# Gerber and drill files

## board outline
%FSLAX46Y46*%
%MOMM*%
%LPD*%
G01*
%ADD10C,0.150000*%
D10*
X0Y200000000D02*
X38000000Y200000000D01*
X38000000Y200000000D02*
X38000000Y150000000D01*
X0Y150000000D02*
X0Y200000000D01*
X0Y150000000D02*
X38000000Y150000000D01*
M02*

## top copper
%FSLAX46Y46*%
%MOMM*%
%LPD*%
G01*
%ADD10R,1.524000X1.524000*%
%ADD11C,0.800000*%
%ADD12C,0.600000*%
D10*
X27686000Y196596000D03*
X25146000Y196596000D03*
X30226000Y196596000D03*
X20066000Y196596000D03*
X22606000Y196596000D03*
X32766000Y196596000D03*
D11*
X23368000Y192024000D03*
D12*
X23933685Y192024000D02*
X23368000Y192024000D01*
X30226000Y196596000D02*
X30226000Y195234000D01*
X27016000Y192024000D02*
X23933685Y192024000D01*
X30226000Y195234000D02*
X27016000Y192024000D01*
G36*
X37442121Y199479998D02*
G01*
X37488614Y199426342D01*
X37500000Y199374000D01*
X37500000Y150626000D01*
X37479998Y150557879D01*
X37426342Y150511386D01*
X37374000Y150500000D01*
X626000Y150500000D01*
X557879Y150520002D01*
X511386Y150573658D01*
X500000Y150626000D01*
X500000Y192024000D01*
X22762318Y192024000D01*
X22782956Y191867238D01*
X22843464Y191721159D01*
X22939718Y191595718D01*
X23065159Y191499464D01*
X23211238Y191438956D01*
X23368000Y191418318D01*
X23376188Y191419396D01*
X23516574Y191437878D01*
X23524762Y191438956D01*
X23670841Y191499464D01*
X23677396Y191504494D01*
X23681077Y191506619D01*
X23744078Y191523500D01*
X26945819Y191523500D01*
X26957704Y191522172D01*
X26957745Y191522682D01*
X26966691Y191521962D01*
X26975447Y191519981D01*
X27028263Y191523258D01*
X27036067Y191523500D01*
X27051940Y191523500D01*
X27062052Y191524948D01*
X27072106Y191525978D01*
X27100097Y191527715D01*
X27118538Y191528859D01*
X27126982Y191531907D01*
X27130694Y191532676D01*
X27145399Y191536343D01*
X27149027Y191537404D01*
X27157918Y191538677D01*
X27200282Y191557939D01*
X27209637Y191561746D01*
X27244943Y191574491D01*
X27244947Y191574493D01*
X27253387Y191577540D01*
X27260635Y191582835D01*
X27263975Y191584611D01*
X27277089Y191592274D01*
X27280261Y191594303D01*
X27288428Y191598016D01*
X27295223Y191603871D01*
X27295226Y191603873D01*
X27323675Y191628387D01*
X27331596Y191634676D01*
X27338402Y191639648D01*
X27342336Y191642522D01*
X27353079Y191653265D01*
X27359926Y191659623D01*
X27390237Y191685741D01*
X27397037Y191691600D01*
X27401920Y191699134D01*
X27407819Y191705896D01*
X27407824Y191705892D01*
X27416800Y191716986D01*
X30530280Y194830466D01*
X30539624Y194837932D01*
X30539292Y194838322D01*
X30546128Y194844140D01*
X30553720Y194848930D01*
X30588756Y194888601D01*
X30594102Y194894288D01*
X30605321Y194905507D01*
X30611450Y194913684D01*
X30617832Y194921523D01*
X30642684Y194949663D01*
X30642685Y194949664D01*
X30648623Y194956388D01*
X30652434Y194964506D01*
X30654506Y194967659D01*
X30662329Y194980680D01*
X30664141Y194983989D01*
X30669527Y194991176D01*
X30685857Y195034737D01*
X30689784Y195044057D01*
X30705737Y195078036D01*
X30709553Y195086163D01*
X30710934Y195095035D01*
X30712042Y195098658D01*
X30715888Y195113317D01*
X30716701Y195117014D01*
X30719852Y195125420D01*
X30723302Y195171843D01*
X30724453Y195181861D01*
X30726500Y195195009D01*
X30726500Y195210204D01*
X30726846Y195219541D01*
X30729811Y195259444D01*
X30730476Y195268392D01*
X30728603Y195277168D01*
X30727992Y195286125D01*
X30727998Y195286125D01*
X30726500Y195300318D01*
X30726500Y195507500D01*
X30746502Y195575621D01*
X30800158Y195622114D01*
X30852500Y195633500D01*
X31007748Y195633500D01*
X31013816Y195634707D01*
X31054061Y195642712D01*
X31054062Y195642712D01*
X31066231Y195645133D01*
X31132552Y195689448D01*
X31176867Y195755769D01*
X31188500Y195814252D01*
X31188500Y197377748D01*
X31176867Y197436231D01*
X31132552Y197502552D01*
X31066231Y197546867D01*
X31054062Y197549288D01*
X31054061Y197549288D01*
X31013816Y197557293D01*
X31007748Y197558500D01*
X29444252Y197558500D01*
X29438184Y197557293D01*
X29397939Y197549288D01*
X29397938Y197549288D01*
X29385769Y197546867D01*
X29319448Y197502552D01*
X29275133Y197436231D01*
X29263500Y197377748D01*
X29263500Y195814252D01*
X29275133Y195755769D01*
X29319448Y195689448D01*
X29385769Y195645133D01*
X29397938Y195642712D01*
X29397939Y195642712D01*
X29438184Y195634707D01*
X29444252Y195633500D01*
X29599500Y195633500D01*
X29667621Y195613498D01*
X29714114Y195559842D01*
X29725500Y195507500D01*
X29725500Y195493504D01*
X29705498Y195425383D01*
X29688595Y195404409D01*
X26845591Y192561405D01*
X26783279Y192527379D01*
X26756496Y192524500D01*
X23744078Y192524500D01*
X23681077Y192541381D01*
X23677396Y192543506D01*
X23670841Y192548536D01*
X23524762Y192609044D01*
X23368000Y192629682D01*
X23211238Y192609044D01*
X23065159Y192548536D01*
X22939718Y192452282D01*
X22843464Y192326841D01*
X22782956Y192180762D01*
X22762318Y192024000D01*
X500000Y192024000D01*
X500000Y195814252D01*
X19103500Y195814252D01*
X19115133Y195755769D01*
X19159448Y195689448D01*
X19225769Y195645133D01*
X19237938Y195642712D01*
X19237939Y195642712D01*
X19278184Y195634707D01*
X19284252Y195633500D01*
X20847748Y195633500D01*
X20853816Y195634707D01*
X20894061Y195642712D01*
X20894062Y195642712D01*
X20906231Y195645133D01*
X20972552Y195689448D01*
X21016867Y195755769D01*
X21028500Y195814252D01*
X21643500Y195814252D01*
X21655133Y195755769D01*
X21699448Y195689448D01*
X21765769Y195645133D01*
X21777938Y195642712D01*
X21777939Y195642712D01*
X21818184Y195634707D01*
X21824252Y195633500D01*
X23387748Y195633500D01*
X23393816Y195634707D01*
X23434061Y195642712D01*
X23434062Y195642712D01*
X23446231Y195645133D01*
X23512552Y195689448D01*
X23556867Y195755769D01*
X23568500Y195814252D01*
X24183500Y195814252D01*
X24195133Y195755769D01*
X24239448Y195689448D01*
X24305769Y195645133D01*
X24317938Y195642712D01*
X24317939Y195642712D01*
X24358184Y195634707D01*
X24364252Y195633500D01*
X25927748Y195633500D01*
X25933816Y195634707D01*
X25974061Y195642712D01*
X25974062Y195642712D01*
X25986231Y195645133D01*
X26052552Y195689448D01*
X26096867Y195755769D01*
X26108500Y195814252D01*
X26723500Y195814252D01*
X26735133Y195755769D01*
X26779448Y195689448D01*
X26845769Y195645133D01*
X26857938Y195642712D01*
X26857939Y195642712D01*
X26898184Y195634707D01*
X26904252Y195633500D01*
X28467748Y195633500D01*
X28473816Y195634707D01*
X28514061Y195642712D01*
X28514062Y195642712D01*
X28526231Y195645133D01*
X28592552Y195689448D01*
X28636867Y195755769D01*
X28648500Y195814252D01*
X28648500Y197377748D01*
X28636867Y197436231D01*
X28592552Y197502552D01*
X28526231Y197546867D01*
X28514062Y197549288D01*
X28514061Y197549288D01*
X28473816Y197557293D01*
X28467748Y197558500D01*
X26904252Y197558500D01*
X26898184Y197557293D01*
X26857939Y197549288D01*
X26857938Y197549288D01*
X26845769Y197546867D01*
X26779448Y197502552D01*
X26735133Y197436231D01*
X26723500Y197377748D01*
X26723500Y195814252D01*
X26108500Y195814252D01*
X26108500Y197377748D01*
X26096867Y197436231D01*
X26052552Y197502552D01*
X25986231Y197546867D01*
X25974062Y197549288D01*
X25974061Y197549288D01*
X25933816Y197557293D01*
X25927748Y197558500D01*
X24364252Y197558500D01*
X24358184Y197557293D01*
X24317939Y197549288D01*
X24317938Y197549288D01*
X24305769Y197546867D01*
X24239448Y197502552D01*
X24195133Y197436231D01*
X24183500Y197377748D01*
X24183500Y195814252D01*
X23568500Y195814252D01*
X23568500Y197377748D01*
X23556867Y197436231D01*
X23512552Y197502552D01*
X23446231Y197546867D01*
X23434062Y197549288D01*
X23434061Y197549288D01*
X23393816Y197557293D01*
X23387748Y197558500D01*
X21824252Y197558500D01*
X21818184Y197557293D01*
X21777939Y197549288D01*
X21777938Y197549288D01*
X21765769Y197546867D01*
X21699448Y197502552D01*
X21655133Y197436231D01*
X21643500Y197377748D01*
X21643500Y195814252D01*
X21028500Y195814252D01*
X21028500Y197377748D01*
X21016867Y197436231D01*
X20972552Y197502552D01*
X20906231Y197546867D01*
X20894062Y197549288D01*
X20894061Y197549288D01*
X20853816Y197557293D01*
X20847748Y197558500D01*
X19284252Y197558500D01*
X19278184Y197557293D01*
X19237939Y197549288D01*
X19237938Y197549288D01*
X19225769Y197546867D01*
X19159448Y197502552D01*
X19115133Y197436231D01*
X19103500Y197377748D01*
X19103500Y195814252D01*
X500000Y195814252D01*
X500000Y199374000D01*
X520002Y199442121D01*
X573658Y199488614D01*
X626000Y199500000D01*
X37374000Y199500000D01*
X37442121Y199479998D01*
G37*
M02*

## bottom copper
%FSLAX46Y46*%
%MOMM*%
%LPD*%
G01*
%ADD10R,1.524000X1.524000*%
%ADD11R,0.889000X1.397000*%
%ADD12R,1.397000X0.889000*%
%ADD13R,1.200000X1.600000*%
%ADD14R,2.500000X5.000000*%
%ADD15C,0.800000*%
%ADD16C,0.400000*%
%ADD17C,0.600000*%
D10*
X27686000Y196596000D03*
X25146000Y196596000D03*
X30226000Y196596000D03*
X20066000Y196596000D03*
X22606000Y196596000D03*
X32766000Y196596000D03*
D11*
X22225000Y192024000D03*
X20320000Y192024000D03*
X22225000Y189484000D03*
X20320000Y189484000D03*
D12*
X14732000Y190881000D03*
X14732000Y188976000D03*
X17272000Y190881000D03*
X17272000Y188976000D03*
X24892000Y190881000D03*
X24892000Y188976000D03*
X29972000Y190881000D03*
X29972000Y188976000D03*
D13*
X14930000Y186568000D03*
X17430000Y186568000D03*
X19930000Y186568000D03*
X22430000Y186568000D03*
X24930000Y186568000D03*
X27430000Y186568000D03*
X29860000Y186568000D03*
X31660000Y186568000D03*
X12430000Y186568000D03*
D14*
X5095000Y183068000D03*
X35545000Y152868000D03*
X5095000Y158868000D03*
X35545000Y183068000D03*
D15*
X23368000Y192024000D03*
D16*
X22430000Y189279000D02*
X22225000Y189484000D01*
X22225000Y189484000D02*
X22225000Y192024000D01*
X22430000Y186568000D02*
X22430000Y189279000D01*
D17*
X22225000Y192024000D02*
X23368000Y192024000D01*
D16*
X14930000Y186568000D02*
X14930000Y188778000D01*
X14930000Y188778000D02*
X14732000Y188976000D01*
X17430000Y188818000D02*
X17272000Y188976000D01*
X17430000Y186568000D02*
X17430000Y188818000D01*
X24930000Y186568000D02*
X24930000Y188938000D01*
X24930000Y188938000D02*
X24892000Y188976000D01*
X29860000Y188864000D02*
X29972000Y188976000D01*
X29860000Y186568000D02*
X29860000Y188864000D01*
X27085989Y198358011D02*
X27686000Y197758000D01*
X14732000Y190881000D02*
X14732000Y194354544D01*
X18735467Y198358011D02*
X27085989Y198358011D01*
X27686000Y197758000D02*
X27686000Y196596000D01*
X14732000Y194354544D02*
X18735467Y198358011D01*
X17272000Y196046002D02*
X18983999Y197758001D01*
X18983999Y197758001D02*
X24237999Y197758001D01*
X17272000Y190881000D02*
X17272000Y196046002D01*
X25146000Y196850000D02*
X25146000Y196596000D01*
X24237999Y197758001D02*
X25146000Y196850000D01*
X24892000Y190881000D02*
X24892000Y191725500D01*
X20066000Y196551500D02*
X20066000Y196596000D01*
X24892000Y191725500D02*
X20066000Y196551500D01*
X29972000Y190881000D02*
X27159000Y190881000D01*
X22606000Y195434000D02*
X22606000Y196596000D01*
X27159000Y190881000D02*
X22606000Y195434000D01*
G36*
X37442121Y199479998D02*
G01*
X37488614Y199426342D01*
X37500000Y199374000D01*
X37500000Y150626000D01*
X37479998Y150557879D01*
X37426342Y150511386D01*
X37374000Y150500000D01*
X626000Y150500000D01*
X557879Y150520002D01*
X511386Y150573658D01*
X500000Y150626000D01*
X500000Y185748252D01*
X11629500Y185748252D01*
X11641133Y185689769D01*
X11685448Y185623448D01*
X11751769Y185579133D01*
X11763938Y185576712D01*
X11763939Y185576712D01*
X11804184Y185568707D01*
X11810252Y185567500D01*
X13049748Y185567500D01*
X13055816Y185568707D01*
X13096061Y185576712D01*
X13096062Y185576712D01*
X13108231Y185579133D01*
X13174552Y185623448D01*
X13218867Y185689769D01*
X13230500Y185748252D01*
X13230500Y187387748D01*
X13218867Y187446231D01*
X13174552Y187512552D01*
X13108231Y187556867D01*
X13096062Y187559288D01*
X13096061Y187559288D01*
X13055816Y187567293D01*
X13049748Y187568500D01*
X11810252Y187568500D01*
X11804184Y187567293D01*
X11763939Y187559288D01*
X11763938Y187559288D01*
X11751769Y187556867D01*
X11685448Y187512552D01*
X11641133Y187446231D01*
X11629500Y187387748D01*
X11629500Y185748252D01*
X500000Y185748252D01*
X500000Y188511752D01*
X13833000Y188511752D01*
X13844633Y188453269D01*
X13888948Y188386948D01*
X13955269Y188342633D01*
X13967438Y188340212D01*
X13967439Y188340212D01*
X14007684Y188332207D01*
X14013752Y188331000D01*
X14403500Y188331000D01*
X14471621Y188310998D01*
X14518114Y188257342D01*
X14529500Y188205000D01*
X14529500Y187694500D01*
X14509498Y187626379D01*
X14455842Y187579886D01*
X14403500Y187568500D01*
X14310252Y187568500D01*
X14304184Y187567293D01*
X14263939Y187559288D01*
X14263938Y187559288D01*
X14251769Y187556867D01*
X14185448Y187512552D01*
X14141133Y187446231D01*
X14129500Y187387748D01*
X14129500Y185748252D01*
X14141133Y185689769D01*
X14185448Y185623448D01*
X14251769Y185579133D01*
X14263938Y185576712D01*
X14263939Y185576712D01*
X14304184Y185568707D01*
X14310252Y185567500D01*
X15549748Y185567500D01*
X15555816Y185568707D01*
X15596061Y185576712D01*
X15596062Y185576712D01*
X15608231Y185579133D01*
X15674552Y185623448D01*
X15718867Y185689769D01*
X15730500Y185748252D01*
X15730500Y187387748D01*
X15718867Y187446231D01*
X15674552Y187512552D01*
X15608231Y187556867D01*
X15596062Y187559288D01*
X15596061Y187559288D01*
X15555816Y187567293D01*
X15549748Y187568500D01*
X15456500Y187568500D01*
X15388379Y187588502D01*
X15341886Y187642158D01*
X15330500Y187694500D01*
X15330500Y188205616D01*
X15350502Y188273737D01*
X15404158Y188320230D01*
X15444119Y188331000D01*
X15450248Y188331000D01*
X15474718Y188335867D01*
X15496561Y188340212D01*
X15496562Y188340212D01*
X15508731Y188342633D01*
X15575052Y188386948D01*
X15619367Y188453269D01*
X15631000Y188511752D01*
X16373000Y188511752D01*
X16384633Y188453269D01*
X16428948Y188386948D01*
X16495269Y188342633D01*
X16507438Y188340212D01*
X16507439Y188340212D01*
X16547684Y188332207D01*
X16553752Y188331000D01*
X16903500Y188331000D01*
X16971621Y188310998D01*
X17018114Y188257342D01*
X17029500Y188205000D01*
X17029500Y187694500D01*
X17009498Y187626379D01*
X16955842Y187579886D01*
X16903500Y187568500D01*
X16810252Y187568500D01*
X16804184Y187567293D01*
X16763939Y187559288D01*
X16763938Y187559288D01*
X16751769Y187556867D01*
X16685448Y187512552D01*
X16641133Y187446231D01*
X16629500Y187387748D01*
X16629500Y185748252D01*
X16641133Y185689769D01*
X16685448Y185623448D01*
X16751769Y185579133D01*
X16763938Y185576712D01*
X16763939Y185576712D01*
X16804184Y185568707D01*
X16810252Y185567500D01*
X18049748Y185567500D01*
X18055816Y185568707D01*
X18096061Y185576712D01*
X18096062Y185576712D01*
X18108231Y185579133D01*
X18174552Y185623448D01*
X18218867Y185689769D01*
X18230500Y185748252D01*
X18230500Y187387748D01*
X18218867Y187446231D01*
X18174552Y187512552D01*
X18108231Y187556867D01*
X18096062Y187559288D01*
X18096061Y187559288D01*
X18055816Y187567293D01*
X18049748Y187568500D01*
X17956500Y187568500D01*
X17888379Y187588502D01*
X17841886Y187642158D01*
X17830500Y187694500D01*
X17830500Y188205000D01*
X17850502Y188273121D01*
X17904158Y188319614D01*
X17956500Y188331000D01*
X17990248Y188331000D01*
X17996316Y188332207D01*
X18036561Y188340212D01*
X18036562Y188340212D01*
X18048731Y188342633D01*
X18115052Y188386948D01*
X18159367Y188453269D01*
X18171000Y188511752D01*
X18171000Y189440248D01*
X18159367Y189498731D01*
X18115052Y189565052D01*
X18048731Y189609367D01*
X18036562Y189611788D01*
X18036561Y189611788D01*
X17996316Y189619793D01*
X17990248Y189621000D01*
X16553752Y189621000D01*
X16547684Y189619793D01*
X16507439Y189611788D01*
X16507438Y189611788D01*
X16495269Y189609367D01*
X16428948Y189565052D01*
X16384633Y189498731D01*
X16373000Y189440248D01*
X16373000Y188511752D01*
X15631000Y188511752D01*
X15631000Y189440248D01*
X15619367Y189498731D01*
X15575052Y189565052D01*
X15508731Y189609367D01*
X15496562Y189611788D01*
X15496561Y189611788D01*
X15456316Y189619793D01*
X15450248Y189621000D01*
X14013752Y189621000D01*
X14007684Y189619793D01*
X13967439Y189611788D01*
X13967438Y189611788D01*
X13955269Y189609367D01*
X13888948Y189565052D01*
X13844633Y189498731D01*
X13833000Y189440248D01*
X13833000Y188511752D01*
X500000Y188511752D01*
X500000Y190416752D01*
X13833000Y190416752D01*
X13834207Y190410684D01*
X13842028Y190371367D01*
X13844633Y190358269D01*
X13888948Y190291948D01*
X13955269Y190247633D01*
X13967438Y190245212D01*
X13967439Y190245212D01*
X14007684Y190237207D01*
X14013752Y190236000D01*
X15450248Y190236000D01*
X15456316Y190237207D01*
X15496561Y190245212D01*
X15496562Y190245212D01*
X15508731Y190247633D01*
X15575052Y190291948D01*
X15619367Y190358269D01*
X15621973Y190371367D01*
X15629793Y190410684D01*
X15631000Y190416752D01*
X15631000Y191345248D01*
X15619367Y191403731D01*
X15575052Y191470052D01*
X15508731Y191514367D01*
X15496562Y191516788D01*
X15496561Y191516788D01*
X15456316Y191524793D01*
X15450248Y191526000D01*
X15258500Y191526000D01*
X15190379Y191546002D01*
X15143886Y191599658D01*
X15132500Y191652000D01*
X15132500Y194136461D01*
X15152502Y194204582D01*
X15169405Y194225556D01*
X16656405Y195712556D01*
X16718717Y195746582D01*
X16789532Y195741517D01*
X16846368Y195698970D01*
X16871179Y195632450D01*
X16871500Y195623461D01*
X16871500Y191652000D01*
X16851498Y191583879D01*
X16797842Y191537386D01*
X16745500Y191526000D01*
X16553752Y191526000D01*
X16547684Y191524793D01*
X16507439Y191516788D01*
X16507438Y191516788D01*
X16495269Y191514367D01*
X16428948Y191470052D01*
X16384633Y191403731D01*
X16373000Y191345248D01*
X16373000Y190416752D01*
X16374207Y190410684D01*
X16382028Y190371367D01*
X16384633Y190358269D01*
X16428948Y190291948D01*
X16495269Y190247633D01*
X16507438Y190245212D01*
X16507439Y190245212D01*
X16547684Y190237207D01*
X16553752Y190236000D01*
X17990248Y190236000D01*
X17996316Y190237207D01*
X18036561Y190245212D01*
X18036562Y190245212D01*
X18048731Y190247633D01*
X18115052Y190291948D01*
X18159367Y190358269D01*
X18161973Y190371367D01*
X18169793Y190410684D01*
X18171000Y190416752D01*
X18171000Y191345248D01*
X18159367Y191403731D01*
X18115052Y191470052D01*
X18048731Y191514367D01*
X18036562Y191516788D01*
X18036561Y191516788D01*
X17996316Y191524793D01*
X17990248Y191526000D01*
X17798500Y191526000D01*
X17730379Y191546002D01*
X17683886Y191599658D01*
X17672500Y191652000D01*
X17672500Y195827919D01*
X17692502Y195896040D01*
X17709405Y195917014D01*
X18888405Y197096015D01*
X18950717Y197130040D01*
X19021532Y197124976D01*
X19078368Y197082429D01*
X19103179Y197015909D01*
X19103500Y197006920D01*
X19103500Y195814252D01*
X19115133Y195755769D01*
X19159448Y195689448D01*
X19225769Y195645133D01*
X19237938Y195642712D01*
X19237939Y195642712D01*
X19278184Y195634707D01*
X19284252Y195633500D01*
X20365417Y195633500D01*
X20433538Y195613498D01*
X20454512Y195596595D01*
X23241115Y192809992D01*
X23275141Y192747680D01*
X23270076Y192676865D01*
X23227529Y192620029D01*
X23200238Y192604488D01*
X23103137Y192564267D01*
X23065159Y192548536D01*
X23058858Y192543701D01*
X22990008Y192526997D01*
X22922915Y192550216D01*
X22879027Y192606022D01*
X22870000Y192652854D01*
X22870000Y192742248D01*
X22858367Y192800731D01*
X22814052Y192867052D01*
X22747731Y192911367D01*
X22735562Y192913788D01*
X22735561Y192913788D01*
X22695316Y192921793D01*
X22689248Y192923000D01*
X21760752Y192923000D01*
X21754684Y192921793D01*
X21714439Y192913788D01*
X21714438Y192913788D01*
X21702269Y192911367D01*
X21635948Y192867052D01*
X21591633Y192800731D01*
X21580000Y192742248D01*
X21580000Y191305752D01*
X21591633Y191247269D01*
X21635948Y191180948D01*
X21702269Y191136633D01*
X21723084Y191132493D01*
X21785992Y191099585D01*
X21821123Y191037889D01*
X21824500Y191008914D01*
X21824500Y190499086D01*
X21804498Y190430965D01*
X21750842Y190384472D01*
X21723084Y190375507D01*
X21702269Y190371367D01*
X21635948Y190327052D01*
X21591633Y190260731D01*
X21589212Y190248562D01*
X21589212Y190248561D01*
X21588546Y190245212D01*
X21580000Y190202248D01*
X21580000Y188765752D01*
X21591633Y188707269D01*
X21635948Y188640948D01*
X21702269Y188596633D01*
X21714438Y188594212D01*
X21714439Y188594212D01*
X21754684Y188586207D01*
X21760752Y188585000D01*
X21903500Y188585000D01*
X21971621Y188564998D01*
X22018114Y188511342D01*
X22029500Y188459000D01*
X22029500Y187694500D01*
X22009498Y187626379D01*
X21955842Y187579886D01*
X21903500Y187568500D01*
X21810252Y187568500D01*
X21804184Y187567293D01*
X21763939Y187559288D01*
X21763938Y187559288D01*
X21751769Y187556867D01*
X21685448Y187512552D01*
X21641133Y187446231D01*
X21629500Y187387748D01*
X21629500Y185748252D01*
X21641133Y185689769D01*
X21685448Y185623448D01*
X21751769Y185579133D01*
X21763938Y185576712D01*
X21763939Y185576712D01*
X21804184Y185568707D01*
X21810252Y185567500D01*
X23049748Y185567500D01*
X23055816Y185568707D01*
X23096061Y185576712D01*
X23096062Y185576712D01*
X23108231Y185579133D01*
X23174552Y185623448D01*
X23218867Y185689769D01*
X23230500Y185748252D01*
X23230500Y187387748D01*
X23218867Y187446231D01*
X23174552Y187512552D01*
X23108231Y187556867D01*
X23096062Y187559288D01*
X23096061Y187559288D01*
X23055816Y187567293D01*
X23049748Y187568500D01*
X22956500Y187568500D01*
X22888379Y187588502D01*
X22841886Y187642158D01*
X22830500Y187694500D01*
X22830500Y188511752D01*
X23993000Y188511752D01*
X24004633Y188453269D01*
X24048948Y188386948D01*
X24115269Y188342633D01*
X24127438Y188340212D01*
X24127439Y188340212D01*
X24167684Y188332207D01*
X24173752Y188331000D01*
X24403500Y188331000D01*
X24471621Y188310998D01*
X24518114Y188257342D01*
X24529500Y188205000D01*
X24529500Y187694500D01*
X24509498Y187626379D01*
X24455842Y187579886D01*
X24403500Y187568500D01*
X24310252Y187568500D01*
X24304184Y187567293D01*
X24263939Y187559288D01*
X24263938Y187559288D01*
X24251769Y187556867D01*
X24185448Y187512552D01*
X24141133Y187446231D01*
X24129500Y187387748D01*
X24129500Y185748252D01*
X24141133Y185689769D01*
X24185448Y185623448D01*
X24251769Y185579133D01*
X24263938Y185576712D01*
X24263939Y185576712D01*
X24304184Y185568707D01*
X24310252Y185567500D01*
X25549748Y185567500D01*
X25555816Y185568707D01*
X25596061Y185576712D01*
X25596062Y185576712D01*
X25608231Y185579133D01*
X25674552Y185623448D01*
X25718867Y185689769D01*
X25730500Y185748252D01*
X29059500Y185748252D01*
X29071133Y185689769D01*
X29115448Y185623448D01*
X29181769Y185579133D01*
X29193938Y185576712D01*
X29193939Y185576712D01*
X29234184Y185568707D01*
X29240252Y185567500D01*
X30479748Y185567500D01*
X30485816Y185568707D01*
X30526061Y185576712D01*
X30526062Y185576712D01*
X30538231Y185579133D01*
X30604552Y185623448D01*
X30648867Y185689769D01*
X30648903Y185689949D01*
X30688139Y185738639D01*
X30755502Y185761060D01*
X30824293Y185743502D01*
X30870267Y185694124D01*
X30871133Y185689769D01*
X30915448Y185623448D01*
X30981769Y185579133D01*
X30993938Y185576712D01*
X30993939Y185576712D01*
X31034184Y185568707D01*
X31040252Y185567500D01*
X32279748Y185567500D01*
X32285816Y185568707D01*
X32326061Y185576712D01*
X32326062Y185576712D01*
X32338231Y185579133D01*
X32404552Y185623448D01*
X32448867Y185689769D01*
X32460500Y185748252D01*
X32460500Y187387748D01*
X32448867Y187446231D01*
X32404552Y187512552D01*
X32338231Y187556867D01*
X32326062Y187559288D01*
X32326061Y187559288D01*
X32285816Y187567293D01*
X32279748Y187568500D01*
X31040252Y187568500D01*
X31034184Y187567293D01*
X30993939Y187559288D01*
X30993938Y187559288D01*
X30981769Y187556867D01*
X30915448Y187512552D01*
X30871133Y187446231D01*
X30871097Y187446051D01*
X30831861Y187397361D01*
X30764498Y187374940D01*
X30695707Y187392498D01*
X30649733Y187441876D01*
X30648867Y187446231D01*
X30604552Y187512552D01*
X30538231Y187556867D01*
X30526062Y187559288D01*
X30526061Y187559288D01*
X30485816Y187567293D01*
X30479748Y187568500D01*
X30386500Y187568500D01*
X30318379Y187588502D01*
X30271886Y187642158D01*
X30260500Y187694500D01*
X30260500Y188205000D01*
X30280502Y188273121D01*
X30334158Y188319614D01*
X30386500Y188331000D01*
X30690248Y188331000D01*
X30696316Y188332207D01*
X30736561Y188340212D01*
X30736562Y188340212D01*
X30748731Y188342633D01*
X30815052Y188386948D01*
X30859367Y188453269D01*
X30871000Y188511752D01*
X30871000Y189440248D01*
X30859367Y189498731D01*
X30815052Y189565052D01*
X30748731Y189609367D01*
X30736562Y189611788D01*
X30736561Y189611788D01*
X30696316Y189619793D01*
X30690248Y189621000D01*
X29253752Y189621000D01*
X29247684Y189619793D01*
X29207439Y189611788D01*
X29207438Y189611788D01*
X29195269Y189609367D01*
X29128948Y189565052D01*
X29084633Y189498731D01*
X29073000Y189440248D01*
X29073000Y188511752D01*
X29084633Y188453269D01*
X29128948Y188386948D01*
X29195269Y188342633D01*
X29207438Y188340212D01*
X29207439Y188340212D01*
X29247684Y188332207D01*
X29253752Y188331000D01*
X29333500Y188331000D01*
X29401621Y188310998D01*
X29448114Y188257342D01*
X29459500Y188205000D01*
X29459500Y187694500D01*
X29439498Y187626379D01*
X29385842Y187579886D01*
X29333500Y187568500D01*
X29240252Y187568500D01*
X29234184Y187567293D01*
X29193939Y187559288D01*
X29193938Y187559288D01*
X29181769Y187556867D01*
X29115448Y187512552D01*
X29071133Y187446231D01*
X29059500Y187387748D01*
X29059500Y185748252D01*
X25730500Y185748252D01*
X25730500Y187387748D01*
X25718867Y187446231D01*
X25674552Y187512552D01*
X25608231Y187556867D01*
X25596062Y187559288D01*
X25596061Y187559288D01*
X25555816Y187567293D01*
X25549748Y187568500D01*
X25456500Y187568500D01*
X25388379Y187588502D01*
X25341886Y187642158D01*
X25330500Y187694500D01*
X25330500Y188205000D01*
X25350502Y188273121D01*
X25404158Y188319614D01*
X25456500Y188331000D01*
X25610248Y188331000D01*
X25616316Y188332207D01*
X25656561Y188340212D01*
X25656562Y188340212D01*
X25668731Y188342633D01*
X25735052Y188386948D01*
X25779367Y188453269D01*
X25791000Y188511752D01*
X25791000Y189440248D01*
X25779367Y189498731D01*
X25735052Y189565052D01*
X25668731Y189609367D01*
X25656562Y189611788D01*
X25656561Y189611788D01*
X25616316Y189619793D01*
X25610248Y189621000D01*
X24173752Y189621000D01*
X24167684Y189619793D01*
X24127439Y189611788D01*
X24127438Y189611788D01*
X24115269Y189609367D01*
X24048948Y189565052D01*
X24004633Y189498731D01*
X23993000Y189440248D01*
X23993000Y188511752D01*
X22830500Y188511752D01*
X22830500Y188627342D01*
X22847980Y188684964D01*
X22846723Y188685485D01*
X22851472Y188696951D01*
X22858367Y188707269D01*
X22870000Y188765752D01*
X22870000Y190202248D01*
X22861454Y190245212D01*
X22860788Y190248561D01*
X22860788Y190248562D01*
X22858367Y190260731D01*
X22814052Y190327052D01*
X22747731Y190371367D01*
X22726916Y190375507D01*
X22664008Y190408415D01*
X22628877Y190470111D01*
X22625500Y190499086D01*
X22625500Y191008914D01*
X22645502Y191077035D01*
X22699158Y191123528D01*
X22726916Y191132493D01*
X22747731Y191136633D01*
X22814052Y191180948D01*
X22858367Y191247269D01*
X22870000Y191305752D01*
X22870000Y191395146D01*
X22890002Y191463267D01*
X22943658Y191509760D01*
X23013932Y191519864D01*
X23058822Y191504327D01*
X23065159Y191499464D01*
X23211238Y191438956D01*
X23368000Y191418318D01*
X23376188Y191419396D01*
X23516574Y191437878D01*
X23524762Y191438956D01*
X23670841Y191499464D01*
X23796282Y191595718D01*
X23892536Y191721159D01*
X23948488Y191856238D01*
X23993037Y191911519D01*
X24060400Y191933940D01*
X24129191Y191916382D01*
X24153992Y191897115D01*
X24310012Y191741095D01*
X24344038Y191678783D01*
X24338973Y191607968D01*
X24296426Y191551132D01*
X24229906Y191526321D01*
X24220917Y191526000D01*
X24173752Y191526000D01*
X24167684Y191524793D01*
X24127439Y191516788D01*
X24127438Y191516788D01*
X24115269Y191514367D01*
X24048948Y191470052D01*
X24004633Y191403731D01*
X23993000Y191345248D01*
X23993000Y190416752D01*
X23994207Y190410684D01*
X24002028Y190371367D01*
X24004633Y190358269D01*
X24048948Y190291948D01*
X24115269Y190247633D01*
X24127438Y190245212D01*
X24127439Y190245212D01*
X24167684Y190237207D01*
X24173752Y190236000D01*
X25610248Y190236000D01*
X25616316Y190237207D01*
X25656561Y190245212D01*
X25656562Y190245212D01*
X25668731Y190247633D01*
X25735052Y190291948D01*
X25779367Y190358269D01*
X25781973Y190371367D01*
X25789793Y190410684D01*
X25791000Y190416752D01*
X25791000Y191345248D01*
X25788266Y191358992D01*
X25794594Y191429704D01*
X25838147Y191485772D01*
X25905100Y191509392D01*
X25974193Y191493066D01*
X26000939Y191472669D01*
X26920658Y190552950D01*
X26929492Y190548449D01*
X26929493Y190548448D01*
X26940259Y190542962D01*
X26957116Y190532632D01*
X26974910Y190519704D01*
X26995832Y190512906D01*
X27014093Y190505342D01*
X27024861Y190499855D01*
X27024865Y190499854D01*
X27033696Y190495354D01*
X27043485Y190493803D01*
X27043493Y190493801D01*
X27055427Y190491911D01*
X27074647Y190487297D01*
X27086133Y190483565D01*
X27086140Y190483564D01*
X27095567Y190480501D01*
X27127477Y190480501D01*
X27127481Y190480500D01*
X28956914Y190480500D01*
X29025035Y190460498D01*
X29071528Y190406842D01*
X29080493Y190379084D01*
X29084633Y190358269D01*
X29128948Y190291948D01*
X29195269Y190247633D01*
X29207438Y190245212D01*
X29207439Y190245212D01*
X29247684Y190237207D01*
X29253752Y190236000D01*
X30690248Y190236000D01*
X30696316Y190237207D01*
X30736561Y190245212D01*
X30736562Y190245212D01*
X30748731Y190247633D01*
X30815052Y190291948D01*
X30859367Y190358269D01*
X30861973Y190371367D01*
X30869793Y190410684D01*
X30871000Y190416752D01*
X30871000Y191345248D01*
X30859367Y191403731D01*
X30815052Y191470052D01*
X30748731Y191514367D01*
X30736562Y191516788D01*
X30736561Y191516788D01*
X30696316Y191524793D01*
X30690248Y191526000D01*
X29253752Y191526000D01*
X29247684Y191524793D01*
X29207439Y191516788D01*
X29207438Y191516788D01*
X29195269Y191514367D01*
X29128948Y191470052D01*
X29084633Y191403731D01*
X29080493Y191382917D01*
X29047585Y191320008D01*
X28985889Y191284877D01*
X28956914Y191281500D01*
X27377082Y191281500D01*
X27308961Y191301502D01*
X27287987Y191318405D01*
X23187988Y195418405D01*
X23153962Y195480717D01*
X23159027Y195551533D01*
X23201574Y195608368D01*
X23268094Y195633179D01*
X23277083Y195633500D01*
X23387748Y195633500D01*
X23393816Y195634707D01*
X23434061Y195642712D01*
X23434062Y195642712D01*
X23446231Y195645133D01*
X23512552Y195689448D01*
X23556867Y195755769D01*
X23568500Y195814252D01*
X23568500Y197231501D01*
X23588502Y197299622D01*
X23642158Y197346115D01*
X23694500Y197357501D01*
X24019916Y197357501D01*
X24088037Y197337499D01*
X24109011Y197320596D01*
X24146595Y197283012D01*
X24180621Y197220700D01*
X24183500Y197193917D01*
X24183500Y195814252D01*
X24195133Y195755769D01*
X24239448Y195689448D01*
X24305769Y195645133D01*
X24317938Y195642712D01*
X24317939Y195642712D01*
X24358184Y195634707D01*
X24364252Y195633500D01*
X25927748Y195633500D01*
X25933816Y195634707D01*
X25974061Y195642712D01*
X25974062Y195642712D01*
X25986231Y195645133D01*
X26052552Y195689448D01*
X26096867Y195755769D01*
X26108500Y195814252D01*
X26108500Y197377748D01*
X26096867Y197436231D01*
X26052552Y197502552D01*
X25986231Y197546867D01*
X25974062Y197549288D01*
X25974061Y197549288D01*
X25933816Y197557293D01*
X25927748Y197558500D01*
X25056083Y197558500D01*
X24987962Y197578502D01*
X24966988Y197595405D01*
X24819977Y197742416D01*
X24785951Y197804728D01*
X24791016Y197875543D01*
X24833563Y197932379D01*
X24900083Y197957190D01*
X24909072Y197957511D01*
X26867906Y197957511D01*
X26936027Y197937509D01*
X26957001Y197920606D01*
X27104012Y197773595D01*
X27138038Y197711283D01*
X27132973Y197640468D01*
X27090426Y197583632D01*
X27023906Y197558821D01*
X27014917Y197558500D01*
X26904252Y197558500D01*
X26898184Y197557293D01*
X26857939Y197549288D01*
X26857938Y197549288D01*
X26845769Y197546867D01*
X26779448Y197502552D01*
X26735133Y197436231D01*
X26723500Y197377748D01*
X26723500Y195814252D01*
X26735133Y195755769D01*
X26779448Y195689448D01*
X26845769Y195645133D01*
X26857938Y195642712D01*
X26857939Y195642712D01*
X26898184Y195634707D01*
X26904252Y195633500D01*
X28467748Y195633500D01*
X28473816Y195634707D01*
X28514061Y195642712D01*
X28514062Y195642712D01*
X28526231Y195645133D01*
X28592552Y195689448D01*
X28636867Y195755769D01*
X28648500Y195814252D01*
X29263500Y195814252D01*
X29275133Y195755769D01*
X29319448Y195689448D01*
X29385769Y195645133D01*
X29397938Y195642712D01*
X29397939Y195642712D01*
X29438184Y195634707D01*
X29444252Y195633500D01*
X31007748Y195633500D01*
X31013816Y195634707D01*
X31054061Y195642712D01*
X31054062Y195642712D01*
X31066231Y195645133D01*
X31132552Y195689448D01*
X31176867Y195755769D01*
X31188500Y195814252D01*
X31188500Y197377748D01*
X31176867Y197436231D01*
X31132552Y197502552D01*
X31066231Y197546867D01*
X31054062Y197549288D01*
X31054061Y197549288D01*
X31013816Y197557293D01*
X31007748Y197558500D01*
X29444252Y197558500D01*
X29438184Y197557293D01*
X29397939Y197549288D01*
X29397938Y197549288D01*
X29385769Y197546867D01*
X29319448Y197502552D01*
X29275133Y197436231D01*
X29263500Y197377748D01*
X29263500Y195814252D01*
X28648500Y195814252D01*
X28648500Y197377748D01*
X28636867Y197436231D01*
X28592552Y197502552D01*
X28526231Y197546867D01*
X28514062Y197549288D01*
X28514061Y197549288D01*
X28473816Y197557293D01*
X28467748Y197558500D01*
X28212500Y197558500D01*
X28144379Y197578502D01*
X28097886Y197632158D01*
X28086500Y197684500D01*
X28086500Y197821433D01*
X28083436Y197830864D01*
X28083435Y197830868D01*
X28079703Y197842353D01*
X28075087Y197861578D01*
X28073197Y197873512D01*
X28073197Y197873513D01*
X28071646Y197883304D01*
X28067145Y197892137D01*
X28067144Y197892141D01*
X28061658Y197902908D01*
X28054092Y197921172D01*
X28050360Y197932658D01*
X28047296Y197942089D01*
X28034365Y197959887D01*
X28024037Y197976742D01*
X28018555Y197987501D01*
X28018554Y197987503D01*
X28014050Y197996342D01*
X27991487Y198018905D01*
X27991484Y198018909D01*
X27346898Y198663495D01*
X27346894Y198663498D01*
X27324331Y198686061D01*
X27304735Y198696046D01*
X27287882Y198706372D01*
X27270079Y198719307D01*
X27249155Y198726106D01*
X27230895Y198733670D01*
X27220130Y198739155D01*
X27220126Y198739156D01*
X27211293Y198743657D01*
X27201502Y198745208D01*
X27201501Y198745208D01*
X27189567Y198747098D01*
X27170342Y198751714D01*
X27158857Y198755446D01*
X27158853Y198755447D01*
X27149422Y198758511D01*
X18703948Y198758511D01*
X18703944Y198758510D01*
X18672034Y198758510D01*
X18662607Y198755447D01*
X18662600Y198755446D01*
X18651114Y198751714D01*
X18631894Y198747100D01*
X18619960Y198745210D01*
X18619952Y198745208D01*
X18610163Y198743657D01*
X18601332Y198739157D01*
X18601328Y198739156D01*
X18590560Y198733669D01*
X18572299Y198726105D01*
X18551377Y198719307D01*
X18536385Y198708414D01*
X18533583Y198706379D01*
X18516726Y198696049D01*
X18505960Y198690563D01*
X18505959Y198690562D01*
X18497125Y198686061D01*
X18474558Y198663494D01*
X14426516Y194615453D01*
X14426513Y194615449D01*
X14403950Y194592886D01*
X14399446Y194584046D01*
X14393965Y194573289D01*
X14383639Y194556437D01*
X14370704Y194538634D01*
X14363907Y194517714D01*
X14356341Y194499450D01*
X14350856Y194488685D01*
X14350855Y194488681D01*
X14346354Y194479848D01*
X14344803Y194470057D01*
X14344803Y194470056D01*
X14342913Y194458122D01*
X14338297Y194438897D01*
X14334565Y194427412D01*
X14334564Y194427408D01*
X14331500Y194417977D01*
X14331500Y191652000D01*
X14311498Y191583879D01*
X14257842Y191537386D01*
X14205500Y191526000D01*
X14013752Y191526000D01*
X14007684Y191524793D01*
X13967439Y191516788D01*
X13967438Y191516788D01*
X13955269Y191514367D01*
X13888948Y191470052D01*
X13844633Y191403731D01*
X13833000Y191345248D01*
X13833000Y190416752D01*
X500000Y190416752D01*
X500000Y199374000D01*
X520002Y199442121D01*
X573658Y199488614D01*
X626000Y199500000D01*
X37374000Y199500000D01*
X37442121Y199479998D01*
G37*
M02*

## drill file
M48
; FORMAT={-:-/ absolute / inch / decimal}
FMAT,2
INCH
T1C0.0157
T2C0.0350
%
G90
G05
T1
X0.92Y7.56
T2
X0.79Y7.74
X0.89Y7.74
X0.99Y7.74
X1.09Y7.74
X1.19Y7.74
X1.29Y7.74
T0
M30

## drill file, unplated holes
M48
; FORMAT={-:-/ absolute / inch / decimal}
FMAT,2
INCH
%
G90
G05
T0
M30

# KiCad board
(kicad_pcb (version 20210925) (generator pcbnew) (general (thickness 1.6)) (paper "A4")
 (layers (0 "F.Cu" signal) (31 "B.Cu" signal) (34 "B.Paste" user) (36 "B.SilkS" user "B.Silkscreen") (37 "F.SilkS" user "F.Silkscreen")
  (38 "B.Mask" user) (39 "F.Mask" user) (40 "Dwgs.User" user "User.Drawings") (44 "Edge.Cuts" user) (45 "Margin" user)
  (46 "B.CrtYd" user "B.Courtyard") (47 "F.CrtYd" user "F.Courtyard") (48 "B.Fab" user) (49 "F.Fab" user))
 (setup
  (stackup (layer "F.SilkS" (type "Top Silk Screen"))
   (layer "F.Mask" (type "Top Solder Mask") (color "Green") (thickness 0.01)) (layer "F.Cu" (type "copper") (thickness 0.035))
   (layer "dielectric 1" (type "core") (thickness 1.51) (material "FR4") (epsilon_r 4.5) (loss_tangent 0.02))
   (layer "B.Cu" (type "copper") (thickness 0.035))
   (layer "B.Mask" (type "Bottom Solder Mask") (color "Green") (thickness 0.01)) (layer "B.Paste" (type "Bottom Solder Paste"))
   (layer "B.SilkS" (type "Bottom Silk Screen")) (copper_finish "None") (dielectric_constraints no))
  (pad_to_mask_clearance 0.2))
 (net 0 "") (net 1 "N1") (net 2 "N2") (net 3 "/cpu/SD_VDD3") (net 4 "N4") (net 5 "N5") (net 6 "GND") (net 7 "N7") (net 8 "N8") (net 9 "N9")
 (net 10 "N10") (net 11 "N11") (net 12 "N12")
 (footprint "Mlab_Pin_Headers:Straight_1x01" (layer "F.Cu") (at 27.686 -196.596)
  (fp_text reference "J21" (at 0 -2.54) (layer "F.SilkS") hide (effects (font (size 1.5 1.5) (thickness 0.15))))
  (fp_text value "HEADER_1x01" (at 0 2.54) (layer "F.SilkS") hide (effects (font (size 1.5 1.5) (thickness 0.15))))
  (pad "1" thru_hole rect locked (at 0 0) (size 1.524 1.524) (drill 0.889) (layers *.Cu *.Mask "F.SilkS") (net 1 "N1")))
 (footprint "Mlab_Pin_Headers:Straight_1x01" (layer "F.Cu") (at 25.146 -196.596)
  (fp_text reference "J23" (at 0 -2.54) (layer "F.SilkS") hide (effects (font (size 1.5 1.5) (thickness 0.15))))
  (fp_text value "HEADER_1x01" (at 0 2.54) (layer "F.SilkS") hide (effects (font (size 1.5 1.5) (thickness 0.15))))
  (pad "1" thru_hole rect locked (at 0 0) (size 1.524 1.524) (drill 0.889) (layers *.Cu *.Mask "F.SilkS") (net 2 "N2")))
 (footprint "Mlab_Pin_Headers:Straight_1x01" (layer "F.Cu") (at 30.226 -196.596)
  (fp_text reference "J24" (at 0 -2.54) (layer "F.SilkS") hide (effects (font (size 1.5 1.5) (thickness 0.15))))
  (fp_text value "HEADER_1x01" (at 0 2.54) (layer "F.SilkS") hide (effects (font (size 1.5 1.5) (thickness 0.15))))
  (pad "1" thru_hole rect locked (at 0 0) (size 1.524 1.524) (drill 0.889) (layers *.Cu *.Mask "F.SilkS") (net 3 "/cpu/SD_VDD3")))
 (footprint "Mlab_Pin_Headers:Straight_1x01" (layer "F.Cu") (at 20.066 -196.596)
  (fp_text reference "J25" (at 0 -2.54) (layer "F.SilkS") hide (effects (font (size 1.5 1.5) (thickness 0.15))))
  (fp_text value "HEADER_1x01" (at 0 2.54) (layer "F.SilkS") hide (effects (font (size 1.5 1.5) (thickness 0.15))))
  (pad "1" thru_hole rect locked (at 0 0) (size 1.524 1.524) (drill 0.889) (layers *.Cu *.Mask "F.SilkS") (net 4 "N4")))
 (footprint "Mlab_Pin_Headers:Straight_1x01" (layer "F.Cu") (at 22.606 -196.596)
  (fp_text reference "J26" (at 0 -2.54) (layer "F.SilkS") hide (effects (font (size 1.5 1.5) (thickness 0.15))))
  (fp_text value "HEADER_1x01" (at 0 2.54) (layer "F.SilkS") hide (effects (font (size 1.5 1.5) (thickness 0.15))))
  (pad "1" thru_hole rect locked (at 0 0) (size 1.524 1.524) (drill 0.889) (layers *.Cu *.Mask "F.SilkS") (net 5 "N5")))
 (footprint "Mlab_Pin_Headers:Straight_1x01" (layer "F.Cu") (at 32.766 -196.596 90)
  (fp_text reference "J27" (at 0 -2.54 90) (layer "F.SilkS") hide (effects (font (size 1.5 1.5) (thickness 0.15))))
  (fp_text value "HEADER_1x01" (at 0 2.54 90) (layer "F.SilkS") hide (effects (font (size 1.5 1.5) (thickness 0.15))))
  (pad "1" thru_hole rect locked (at 0 0 90) (size 1.524 1.524) (drill 0.889) (layers *.Cu *.Mask "F.SilkS") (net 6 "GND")))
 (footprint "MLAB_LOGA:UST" (layer "F.Cu") (at 18.415 -175.133)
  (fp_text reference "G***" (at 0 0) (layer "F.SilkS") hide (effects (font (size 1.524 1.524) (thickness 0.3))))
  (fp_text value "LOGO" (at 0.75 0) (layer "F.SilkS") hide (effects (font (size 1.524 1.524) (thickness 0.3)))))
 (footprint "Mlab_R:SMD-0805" (layer "B.Cu") (at 21.2725 -192.024 180)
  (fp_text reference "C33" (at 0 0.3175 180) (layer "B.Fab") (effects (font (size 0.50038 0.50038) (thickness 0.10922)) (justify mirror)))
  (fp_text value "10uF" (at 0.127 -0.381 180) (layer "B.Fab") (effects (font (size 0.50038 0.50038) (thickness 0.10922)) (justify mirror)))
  (pad "1" smd rect locked (at -0.9525 0 180) (size 0.889 1.397) (layers "B.Cu" "B.Paste" "B.Mask") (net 3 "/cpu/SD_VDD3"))
  (pad "2" smd rect locked (at 0.9525 0 180) (size 0.889 1.397) (layers "B.Cu" "B.Paste" "B.Mask") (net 6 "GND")))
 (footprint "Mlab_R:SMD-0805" (layer "B.Cu") (at 21.2725 -189.484 180)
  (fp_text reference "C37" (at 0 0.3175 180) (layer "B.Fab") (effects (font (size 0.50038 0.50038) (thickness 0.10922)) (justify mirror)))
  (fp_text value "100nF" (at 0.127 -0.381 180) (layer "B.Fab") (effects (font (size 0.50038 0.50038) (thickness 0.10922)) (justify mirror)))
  (pad "1" smd rect locked (at -0.9525 0 180) (size 0.889 1.397) (layers "B.Cu" "B.Paste" "B.Mask") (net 3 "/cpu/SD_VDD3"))
  (pad "2" smd rect locked (at 0.9525 0 180) (size 0.889 1.397) (layers "B.Cu" "B.Paste" "B.Mask") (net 6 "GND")))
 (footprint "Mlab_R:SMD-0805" (layer "B.Cu") (at 14.732 -189.9285 -90)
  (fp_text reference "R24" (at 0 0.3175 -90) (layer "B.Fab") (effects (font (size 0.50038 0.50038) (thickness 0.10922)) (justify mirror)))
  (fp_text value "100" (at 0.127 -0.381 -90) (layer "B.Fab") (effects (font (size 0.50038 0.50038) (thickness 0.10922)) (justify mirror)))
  (pad "1" smd rect locked (at -0.9525 0 270) (size 0.889 1.397) (layers "B.Cu" "B.Paste" "B.Mask") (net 1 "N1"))
  (pad "2" smd rect locked (at 0.9525 0 270) (size 0.889 1.397) (layers "B.Cu" "B.Paste" "B.Mask") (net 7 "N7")))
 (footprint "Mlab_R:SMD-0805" (layer "B.Cu") (at 17.272 -189.9285 -90)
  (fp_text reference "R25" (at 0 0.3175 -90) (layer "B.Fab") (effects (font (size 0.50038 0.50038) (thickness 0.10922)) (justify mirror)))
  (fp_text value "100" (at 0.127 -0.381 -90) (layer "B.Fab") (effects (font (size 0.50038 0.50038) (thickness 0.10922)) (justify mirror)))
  (pad "1" smd rect locked (at -0.9525 0 270) (size 0.889 1.397) (layers "B.Cu" "B.Paste" "B.Mask") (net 2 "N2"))
  (pad "2" smd rect locked (at 0.9525 0 270) (size 0.889 1.397) (layers "B.Cu" "B.Paste" "B.Mask") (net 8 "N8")))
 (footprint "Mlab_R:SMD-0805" (layer "B.Cu") (at 24.892 -189.9285 -90)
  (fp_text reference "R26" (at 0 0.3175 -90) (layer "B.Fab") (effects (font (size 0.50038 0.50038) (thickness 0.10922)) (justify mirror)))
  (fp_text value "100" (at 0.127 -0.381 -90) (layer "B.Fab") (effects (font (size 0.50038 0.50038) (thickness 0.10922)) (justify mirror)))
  (pad "1" smd rect locked (at -0.9525 0 270) (size 0.889 1.397) (layers "B.Cu" "B.Paste" "B.Mask") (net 4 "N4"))
  (pad "2" smd rect locked (at 0.9525 0 270) (size 0.889 1.397) (layers "B.Cu" "B.Paste" "B.Mask") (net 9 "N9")))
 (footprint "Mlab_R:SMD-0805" (layer "B.Cu") (at 29.972 -189.9285 -90)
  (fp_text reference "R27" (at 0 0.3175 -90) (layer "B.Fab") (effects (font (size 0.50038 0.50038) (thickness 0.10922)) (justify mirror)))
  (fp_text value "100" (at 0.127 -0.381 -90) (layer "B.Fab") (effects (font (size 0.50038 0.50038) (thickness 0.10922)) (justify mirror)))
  (pad "1" smd rect locked (at -0.9525 0 270) (size 0.889 1.397) (layers "B.Cu" "B.Paste" "B.Mask") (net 5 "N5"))
  (pad "2" smd rect locked (at 0.9525 0 270) (size 0.889 1.397) (layers "B.Cu" "B.Paste" "B.Mask") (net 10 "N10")))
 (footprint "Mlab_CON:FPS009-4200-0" (layer "B.Cu") (at 20.32 -150.368 -90)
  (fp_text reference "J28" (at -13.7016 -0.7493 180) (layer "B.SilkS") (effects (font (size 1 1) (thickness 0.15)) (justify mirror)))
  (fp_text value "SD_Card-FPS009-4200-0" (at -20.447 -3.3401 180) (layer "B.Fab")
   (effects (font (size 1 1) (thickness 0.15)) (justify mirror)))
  (pad "1" smd rect locked (at -36.2 5.39 90) (size 1.6 1.2) (layers "B.Cu" "B.Paste" "B.Mask") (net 7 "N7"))
  (pad "2" smd rect locked (at -36.2 2.89 90) (size 1.6 1.2) (layers "B.Cu" "B.Paste" "B.Mask") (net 8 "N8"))
  (pad "3" smd rect locked (at -36.2 0.39 90) (size 1.6 1.2) (layers "B.Cu" "B.Paste" "B.Mask") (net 6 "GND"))
  (pad "4" smd rect locked (at -36.2 -2.11 90) (size 1.6 1.2) (layers "B.Cu" "B.Paste" "B.Mask") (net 3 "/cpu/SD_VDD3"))
  (pad "5" smd rect locked (at -36.2 -4.61 90) (size 1.6 1.2) (layers "B.Cu" "B.Paste" "B.Mask") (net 9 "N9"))
  (pad "6" smd rect locked (at -36.2 -7.11 90) (size 1.6 1.2) (layers "B.Cu" "B.Paste" "B.Mask") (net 6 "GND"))
  (pad "7" smd rect locked (at -36.2 -9.54 90) (size 1.6 1.2) (layers "B.Cu" "B.Paste" "B.Mask") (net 10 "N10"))
  (pad "8" smd rect locked (at -36.2 -11.34 90) (size 1.6 1.2) (layers "B.Cu" "B.Paste" "B.Mask") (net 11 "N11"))
  (pad "9" smd rect locked (at -36.2 7.89 180) (size 1.2 1.6) (layers "B.Cu" "B.Paste" "B.Mask") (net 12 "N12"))
  (pad "12" smd rect locked (at -32.7 15.225 90) (size 5 2.5) (layers "B.Cu" "B.Paste" "B.Mask") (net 6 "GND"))
  (pad "12" smd rect locked (at -2.5 -15.225 90) (size 5 2.5) (layers "B.Cu" "B.Paste" "B.Mask") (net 6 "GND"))
  (pad "12" smd rect locked (at -8.5 15.225 90) (size 5 2.5) (layers "B.Cu" "B.Paste" "B.Mask") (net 6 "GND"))
  (pad "12" smd rect locked (at -32.7 -15.225 90) (size 5 2.5) (layers "B.Cu" "B.Paste" "B.Mask") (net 6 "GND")))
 (gr_line (start 0 -200) (end 38 -200) (layer "Edge.Cuts") (width 0.15))
 (gr_line (start 38 -200) (end 38 -150) (layer "Edge.Cuts") (width 0.15))
 (gr_line (start 0 -150) (end 0 -200) (layer "Edge.Cuts") (width 0.15))
 (gr_line (start 0 -150) (end 38 -150) (layer "Edge.Cuts") (width 0.15))
 (segment (start 23.933685 -192.024) (end 23.368 -192.024) (width 0.6) (layer "F.Cu") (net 3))
 (segment (start 30.226 -196.596) (end 30.226 -195.234) (width 0.6) (layer "F.Cu") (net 3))
 (segment (start 27.016 -192.024) (end 23.933685 -192.024) (width 0.6) (layer "F.Cu") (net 3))
 (segment (start 30.226 -195.234) (end 27.016 -192.024) (width 0.6) (layer "F.Cu") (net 3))
 (via (at 23.368 -192.024) (size 0.8) (drill 0.4) (layers "F.Cu" "B.Cu") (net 3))
 (segment (start 22.43 -189.279) (end 22.225 -189.484) (width 0.4) (layer "B.Cu") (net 3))
 (segment (start 22.225 -189.484) (end 22.225 -192.024) (width 0.4) (layer "B.Cu") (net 3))
 (segment (start 22.43 -186.568) (end 22.43 -189.279) (width 0.4) (layer "B.Cu") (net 3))
 (segment (start 22.225 -192.024) (end 23.368 -192.024) (width 0.6) (layer "B.Cu") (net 3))
 (segment (start 14.93 -186.568) (end 14.93 -188.778) (width 0.4) (layer "B.Cu") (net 7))
 (segment (start 14.93 -188.778) (end 14.732 -188.976) (width 0.4) (layer "B.Cu") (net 7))
 (segment (start 17.43 -188.818) (end 17.272 -188.976) (width 0.4) (layer "B.Cu") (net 8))
 (segment (start 17.43 -186.568) (end 17.43 -188.818) (width 0.4) (layer "B.Cu") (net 8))
 (segment (start 24.93 -186.568) (end 24.93 -188.938) (width 0.4) (layer "B.Cu") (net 9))
 (segment (start 24.93 -188.938) (end 24.892 -188.976) (width 0.4) (layer "B.Cu") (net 9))
 (segment (start 29.86 -188.864) (end 29.972 -188.976) (width 0.4) (layer "B.Cu") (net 10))
 (segment (start 29.86 -186.568) (end 29.86 -188.864) (width 0.4) (layer "B.Cu") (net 10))
 (segment (start 27.085989 -198.358011) (end 27.686 -197.758) (width 0.4) (layer "B.Cu") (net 1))
 (segment (start 14.732 -190.881) (end 14.732 -194.354544) (width 0.4) (layer "B.Cu") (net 1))
 (segment (start 18.735467 -198.358011) (end 27.085989 -198.358011) (width 0.4) (layer "B.Cu") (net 1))
 (segment (start 27.686 -197.758) (end 27.686 -196.596) (width 0.4) (layer "B.Cu") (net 1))
 (segment (start 14.732 -194.354544) (end 18.735467 -198.358011) (width 0.4) (layer "B.Cu") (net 1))
 (segment (start 17.272 -196.046002) (end 18.983999 -197.758001) (width 0.4) (layer "B.Cu") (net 2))
 (segment (start 18.983999 -197.758001) (end 24.237999 -197.758001) (width 0.4) (layer "B.Cu") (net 2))
 (segment (start 17.272 -190.881) (end 17.272 -196.046002) (width 0.4) (layer "B.Cu") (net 2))
 (segment (start 25.146 -196.85) (end 25.146 -196.596) (width 0.4) (layer "B.Cu") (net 2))
 (segment (start 24.237999 -197.758001) (end 25.146 -196.85) (width 0.4) (layer "B.Cu") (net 2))
 (segment (start 24.892 -190.881) (end 24.892 -191.7255) (width 0.4) (layer "B.Cu") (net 4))
 (segment (start 20.066 -196.5515) (end 20.066 -196.596) (width 0.4) (layer "B.Cu") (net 4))
 (segment (start 24.892 -191.7255) (end 20.066 -196.5515) (width 0.4) (layer "B.Cu") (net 4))
 (segment (start 29.972 -190.881) (end 27.159 -190.881) (width 0.4) (layer "B.Cu") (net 5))
 (segment (start 22.606 -195.434) (end 22.606 -196.596) (width 0.4) (layer "B.Cu") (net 5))
 (segment (start 27.159 -190.881) (end 22.606 -195.434) (width 0.4) (layer "B.Cu") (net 5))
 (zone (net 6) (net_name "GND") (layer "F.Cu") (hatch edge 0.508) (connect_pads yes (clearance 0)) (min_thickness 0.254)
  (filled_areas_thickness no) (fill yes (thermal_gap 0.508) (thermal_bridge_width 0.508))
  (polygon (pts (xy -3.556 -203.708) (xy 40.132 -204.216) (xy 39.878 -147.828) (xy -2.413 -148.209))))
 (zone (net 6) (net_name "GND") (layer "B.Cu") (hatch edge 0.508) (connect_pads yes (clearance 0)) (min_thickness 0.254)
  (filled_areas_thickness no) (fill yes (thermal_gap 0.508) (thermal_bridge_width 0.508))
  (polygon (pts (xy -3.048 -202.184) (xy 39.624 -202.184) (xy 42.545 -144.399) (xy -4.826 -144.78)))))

